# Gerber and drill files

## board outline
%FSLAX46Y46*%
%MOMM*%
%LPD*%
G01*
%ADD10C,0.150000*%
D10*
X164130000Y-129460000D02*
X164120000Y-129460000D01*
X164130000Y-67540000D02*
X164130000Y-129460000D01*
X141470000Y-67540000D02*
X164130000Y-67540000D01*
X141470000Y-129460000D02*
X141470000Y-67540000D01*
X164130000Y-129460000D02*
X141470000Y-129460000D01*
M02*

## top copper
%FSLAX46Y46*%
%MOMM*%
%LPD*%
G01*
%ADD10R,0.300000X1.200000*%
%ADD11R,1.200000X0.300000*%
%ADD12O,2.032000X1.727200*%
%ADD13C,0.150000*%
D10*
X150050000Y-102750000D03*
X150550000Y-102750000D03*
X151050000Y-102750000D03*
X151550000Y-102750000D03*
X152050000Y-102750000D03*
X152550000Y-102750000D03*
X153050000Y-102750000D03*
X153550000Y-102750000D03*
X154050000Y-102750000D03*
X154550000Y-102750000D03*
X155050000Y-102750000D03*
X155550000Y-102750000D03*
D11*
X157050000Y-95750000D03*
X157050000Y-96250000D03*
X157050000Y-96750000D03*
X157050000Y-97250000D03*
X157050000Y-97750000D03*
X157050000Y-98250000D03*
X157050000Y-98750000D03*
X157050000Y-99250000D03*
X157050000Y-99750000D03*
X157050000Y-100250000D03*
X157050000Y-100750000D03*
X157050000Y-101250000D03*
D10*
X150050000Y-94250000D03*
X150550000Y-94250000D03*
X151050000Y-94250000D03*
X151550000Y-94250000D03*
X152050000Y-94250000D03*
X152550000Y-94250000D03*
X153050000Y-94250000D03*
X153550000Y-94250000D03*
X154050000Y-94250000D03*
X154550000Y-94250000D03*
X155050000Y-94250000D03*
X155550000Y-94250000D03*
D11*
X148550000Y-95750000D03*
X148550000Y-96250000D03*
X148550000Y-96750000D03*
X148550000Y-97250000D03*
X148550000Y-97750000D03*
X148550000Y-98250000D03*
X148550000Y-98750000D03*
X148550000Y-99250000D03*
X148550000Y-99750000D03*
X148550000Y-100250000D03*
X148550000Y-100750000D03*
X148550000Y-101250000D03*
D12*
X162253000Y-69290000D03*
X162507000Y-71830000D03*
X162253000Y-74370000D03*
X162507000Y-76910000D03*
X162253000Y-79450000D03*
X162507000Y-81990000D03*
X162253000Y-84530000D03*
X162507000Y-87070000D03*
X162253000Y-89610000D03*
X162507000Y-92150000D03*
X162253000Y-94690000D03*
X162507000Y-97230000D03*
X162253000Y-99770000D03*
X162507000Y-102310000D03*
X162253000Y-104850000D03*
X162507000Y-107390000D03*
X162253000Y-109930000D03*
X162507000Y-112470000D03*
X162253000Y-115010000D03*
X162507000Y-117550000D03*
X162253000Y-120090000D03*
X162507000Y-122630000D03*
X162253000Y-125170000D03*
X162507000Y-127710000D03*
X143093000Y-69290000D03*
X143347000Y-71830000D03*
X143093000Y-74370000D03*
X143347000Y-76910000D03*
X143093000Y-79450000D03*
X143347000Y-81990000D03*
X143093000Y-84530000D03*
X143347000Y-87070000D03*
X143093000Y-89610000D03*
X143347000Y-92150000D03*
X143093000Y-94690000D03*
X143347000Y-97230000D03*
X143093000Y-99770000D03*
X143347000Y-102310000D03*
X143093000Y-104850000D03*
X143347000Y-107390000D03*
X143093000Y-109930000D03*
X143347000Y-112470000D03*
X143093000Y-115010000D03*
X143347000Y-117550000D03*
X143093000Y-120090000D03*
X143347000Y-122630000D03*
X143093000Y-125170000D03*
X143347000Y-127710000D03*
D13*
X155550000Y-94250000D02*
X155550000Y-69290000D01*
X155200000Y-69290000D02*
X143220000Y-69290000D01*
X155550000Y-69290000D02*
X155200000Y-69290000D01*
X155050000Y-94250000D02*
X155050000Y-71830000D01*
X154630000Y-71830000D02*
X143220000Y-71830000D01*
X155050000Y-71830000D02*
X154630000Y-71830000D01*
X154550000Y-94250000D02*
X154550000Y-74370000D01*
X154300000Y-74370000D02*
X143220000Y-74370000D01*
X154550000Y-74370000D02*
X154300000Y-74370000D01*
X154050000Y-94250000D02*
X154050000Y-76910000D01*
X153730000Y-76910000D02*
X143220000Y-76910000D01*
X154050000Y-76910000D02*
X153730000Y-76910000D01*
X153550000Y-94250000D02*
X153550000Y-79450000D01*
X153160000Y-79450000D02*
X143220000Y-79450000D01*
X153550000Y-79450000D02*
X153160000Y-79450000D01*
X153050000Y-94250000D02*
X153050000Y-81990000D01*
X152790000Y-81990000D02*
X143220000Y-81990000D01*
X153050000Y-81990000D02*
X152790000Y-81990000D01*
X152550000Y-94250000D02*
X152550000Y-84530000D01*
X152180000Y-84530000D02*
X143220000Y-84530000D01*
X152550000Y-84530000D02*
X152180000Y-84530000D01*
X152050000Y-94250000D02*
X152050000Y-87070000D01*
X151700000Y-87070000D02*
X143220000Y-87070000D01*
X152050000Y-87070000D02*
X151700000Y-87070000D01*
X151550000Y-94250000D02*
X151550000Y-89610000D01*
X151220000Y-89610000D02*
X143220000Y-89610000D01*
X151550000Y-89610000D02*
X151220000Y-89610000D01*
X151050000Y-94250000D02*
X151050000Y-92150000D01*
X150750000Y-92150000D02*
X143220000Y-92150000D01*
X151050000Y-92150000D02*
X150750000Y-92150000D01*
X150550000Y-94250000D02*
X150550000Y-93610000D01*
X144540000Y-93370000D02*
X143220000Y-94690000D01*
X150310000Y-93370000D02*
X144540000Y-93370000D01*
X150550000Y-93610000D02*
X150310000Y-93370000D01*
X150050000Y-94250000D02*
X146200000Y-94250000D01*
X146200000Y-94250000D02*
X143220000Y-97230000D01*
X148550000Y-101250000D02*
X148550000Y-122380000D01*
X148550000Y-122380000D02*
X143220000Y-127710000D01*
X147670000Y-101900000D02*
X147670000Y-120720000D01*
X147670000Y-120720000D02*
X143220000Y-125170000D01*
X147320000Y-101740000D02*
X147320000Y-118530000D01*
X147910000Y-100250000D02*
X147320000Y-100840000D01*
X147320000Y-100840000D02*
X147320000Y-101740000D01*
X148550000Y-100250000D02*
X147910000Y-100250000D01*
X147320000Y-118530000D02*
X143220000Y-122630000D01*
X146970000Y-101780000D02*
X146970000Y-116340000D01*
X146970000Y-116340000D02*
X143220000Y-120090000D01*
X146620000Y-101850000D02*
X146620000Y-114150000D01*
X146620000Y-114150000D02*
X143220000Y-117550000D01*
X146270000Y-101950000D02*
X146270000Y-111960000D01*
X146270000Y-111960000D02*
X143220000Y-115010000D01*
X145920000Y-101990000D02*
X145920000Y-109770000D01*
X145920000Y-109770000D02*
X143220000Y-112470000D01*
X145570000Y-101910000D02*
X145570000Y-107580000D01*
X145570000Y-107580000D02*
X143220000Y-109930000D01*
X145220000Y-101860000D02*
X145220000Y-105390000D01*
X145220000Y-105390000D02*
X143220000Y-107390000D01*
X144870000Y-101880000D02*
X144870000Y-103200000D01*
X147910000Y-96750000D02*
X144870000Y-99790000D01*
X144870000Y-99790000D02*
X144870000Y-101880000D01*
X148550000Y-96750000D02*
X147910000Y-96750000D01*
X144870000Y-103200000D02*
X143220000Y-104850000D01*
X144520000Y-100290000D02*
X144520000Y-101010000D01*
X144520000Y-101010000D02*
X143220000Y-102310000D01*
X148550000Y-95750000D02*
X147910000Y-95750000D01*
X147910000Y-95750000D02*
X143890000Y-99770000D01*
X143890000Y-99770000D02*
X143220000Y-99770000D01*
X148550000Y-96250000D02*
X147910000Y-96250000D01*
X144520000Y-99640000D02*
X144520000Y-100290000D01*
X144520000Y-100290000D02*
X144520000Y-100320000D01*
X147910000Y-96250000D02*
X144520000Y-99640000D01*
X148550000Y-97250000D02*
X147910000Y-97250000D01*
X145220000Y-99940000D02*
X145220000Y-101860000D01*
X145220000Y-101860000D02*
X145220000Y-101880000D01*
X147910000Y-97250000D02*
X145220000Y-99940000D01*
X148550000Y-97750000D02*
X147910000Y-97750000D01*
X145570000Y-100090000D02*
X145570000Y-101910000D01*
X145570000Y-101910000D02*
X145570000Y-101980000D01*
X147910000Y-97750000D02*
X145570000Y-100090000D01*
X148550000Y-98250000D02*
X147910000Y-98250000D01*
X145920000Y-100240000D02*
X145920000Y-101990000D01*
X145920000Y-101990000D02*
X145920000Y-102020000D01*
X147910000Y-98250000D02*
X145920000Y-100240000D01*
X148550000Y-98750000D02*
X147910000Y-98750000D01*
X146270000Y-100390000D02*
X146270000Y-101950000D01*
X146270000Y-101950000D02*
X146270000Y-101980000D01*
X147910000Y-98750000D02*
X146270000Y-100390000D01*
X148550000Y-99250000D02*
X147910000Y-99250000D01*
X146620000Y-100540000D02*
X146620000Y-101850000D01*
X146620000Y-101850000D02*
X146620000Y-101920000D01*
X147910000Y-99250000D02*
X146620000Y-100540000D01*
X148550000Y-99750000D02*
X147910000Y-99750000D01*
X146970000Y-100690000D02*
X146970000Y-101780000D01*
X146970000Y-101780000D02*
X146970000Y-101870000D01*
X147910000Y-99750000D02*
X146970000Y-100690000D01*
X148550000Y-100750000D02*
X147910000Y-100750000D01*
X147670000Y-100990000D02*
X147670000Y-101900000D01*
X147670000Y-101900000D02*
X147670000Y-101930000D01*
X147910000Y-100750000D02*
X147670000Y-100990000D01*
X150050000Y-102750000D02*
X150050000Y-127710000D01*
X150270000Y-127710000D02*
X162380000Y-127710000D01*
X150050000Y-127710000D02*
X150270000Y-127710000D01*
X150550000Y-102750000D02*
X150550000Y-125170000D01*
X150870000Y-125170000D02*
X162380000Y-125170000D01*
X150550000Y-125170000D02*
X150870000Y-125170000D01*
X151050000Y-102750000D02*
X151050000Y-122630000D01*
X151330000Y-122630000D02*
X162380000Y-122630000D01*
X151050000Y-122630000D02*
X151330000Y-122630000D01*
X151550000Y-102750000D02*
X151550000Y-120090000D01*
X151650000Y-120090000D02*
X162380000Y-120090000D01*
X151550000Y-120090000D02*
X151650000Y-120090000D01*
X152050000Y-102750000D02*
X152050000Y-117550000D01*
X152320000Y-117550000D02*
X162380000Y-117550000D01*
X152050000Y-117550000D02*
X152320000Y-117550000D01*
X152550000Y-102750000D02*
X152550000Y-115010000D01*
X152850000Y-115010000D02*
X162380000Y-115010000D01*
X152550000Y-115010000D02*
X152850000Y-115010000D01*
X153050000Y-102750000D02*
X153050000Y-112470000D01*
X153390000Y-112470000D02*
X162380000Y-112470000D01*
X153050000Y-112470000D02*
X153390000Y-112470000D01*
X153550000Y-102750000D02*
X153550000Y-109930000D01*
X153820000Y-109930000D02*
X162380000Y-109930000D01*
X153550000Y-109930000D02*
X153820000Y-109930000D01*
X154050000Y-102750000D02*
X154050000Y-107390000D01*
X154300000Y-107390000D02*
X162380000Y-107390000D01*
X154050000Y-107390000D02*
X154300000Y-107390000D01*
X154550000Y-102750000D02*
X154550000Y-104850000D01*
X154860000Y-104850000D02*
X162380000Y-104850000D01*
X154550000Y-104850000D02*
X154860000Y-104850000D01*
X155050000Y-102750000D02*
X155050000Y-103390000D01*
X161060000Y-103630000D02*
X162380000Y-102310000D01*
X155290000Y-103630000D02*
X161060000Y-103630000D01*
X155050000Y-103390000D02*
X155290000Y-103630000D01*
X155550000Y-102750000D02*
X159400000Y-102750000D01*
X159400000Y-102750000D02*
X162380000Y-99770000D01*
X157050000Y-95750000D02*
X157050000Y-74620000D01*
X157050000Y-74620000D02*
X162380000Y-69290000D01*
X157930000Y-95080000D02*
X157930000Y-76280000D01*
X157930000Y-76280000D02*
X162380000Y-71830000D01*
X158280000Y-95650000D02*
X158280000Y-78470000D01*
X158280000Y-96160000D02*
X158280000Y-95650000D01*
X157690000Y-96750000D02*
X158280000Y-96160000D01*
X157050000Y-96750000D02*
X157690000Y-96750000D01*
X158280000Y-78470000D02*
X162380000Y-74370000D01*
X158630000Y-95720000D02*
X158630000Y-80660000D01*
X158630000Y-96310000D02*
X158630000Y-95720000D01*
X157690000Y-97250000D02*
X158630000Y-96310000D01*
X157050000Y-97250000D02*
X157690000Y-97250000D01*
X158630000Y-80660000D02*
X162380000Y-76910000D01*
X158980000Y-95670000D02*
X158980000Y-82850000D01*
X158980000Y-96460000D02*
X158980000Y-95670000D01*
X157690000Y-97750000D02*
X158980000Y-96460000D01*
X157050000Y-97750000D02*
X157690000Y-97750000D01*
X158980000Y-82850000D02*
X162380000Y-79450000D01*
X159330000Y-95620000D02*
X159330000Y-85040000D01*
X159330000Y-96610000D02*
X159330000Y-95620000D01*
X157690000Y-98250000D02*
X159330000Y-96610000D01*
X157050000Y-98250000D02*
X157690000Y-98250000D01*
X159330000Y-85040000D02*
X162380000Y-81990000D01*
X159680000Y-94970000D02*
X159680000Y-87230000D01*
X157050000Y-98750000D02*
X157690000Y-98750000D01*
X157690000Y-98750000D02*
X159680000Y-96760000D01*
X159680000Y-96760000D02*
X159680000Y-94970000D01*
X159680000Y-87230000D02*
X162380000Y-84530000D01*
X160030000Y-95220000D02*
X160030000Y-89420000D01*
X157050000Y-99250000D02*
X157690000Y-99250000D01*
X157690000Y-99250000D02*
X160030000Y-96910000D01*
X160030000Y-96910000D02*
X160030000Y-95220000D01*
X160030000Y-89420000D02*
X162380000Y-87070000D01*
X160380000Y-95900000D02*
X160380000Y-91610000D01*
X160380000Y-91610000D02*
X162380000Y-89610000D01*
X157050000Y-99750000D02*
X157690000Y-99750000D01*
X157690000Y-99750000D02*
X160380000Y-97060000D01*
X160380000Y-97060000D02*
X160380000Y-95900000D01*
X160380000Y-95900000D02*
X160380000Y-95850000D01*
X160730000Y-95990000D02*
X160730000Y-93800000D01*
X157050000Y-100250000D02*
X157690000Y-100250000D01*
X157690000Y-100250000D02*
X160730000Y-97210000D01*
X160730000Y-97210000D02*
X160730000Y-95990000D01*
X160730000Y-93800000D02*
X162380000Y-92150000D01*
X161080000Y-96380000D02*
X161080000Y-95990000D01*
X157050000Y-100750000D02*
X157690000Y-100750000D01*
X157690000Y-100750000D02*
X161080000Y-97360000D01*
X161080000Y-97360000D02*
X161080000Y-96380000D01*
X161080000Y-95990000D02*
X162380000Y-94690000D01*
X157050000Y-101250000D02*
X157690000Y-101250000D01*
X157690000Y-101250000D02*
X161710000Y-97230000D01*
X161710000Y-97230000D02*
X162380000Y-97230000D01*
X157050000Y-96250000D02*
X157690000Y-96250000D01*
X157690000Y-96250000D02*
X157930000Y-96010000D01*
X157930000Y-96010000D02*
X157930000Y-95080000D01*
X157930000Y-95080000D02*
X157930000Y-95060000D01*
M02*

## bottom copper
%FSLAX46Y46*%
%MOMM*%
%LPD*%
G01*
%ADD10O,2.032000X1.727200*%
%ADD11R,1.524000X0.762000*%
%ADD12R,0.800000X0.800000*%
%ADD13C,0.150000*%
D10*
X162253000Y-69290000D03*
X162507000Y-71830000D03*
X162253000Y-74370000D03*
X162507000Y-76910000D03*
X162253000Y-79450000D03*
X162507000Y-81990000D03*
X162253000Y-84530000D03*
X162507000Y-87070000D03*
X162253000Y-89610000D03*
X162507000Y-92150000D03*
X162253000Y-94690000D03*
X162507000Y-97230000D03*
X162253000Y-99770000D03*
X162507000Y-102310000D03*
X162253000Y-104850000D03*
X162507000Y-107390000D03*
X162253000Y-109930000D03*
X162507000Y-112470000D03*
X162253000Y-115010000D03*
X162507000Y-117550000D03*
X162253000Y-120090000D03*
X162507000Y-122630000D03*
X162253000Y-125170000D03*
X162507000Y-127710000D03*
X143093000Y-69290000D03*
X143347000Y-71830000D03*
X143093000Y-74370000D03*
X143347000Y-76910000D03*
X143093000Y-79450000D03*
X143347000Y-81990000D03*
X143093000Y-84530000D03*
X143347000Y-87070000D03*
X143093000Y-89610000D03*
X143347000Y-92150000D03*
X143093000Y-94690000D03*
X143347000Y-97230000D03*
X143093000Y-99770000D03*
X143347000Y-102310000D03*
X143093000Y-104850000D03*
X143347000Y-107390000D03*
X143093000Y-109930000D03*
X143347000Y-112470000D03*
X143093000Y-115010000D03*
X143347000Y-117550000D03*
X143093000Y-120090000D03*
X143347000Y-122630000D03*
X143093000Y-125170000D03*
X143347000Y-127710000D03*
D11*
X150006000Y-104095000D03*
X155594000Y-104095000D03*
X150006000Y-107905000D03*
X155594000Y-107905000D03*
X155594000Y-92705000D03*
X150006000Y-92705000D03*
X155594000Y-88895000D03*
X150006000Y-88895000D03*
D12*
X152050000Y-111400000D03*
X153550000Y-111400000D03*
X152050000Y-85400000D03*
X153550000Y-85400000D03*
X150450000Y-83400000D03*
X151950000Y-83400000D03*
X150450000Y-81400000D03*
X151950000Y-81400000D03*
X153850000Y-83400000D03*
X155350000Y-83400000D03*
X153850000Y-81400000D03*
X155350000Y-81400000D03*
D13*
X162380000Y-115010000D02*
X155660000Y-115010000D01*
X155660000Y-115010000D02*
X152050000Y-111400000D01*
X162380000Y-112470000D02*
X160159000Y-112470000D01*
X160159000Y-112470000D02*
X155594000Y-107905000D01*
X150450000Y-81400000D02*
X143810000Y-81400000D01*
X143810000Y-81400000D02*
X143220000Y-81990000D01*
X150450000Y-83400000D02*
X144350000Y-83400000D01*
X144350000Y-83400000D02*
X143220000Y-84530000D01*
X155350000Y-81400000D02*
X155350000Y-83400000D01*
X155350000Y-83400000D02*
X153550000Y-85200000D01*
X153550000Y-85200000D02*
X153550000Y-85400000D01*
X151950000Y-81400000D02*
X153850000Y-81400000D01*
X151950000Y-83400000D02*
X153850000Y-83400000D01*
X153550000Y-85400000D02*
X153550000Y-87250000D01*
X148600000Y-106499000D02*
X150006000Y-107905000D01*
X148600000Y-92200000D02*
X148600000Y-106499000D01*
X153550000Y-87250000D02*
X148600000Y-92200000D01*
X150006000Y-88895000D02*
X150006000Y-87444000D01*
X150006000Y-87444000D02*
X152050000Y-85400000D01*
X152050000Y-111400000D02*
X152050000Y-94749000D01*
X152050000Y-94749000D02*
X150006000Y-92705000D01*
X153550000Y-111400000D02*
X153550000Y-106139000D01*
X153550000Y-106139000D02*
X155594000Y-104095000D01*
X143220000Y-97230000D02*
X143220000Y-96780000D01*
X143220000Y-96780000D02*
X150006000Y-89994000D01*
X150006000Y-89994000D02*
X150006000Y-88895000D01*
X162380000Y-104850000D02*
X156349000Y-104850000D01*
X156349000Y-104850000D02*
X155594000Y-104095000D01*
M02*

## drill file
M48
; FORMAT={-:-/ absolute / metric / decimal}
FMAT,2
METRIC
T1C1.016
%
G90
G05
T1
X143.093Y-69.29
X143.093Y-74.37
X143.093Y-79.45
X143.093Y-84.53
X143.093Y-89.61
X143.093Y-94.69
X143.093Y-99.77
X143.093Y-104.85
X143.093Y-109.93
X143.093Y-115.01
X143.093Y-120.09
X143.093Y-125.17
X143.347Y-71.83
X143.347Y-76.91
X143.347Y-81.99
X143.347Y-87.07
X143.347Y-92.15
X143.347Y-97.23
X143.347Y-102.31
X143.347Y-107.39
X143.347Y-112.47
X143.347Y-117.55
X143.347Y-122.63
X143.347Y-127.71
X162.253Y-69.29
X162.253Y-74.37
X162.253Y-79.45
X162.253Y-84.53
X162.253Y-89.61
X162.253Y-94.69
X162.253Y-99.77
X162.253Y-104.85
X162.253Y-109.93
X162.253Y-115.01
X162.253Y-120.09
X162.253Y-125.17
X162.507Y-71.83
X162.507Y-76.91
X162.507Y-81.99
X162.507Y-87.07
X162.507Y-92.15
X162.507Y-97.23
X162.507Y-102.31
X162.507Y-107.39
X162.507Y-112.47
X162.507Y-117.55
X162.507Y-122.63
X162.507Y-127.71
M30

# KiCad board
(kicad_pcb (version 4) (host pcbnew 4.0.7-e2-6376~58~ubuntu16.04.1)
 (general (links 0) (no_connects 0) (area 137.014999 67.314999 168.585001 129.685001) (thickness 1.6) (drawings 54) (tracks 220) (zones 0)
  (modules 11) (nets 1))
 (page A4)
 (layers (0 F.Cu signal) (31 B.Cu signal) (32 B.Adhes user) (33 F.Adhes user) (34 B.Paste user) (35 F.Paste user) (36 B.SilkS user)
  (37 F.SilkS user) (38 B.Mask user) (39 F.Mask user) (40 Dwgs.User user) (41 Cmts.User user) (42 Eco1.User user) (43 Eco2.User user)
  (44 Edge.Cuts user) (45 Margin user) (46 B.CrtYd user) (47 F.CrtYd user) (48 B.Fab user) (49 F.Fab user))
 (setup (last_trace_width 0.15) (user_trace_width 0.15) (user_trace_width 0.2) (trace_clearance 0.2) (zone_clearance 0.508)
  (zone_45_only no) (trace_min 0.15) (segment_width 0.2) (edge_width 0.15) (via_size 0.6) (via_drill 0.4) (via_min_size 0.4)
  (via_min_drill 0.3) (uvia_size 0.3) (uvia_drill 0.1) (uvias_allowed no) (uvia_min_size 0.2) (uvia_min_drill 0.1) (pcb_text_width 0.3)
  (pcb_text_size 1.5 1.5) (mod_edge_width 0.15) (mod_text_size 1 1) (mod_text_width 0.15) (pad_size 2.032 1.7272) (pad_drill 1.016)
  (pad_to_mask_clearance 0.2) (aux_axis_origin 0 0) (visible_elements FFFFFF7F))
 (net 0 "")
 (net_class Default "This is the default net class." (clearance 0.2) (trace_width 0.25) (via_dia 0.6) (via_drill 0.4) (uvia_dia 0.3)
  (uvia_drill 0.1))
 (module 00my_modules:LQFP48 (layer F.Cu) (at 152.8 98.5)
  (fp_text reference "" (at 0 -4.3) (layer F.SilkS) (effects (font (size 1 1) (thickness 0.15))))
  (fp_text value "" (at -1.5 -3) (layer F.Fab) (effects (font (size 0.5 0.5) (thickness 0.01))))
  (pad 1 smd rect (at -2.75 4.25) (size 0.3 1.2) (layers F.Cu F.Paste F.Mask))
  (pad 2 smd rect (at -2.25 4.25) (size 0.3 1.2) (layers F.Cu F.Paste F.Mask))
  (pad 3 smd rect (at -1.75 4.25) (size 0.3 1.2) (layers F.Cu F.Paste F.Mask))
  (pad 4 smd rect (at -1.25 4.25) (size 0.3 1.2) (layers F.Cu F.Paste F.Mask))
  (pad 5 smd rect (at -0.75 4.25) (size 0.3 1.2) (layers F.Cu F.Paste F.Mask))
  (pad 6 smd rect (at -0.25 4.25) (size 0.3 1.2) (layers F.Cu F.Paste F.Mask))
  (pad 7 smd rect (at 0.25 4.25) (size 0.3 1.2) (layers F.Cu F.Paste F.Mask))
  (pad 8 smd rect (at 0.75 4.25) (size 0.3 1.2) (layers F.Cu F.Paste F.Mask))
  (pad 9 smd rect (at 1.25 4.25) (size 0.3 1.2) (layers F.Cu F.Paste F.Mask))
  (pad 10 smd rect (at 1.75 4.25) (size 0.3 1.2) (layers F.Cu F.Paste F.Mask))
  (pad 11 smd rect (at 2.25 4.25) (size 0.3 1.2) (layers F.Cu F.Paste F.Mask))
  (pad 12 smd rect (at 2.75 4.25) (size 0.3 1.2) (layers F.Cu F.Paste F.Mask))
  (pad 24 smd rect (at 4.25 -2.75) (size 1.2 0.3) (layers F.Cu F.Paste F.Mask))
  (pad 23 smd rect (at 4.25 -2.25) (size 1.2 0.3) (layers F.Cu F.Paste F.Mask))
  (pad 22 smd rect (at 4.25 -1.75) (size 1.2 0.3) (layers F.Cu F.Paste F.Mask))
  (pad 21 smd rect (at 4.25 -1.25) (size 1.2 0.3) (layers F.Cu F.Paste F.Mask))
  (pad 20 smd rect (at 4.25 -0.75) (size 1.2 0.3) (layers F.Cu F.Paste F.Mask))
  (pad 19 smd rect (at 4.25 -0.25) (size 1.2 0.3) (layers F.Cu F.Paste F.Mask))
  (pad 18 smd rect (at 4.25 0.25) (size 1.2 0.3) (layers F.Cu F.Paste F.Mask))
  (pad 17 smd rect (at 4.25 0.75) (size 1.2 0.3) (layers F.Cu F.Paste F.Mask))
  (pad 16 smd rect (at 4.25 1.25) (size 1.2 0.3) (layers F.Cu F.Paste F.Mask))
  (pad 15 smd rect (at 4.25 1.75) (size 1.2 0.3) (layers F.Cu F.Paste F.Mask))
  (pad 14 smd rect (at 4.25 2.25) (size 1.2 0.3) (layers F.Cu F.Paste F.Mask))
  (pad 13 smd rect (at 4.25 2.75) (size 1.2 0.3) (layers F.Cu F.Paste F.Mask))
  (pad 36 smd rect (at -2.75 -4.25) (size 0.3 1.2) (layers F.Cu F.Paste F.Mask))
  (pad 35 smd rect (at -2.25 -4.25) (size 0.3 1.2) (layers F.Cu F.Paste F.Mask))
  (pad 34 smd rect (at -1.75 -4.25) (size 0.3 1.2) (layers F.Cu F.Paste F.Mask))
  (pad 33 smd rect (at -1.25 -4.25) (size 0.3 1.2) (layers F.Cu F.Paste F.Mask))
  (pad 32 smd rect (at -0.75 -4.25) (size 0.3 1.2) (layers F.Cu F.Paste F.Mask))
  (pad 31 smd rect (at -0.25 -4.25) (size 0.3 1.2) (layers F.Cu F.Paste F.Mask))
  (pad 30 smd rect (at 0.25 -4.25) (size 0.3 1.2) (layers F.Cu F.Paste F.Mask))
  (pad 29 smd rect (at 0.75 -4.25) (size 0.3 1.2) (layers F.Cu F.Paste F.Mask))
  (pad 28 smd rect (at 1.25 -4.25) (size 0.3 1.2) (layers F.Cu F.Paste F.Mask))
  (pad 27 smd rect (at 1.75 -4.25) (size 0.3 1.2) (layers F.Cu F.Paste F.Mask))
  (pad 26 smd rect (at 2.25 -4.25) (size 0.3 1.2) (layers F.Cu F.Paste F.Mask))
  (pad 25 smd rect (at 2.75 -4.25) (size 0.3 1.2) (layers F.Cu F.Paste F.Mask))
  (pad 37 smd rect (at -4.25 -2.75) (size 1.2 0.3) (layers F.Cu F.Paste F.Mask))
  (pad 38 smd rect (at -4.25 -2.25) (size 1.2 0.3) (layers F.Cu F.Paste F.Mask))
  (pad 39 smd rect (at -4.25 -1.75) (size 1.2 0.3) (layers F.Cu F.Paste F.Mask))
  (pad 40 smd rect (at -4.25 -1.25) (size 1.2 0.3) (layers F.Cu F.Paste F.Mask))
  (pad 41 smd rect (at -4.25 -0.75) (size 1.2 0.3) (layers F.Cu F.Paste F.Mask))
  (pad 42 smd rect (at -4.25 -0.25) (size 1.2 0.3) (layers F.Cu F.Paste F.Mask))
  (pad 43 smd rect (at -4.25 0.25) (size 1.2 0.3) (layers F.Cu F.Paste F.Mask))
  (pad 44 smd rect (at -4.25 0.75) (size 1.2 0.3) (layers F.Cu F.Paste F.Mask))
  (pad 45 smd rect (at -4.25 1.25) (size 1.2 0.3) (layers F.Cu F.Paste F.Mask))
  (pad 46 smd rect (at -4.25 1.75) (size 1.2 0.3) (layers F.Cu F.Paste F.Mask))
  (pad 47 smd rect (at -4.25 2.25) (size 1.2 0.3) (layers F.Cu F.Paste F.Mask))
  (pad 48 smd rect (at -4.25 2.75) (size 1.2 0.3) (layers F.Cu F.Paste F.Mask)))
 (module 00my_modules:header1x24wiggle (layer F.Cu) (at 162.38 98.5)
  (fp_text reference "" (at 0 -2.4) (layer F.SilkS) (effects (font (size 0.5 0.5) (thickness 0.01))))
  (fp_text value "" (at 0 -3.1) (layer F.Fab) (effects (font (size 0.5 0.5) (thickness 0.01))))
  (pad 24 thru_hole oval (at -0.127 -29.21) (size 2.032 1.7272) (drill 1.016) (layers *.Cu *.Mask F.SilkS))
  (pad 23 thru_hole oval (at 0.127 -26.67) (size 2.032 1.7272) (drill 1.016) (layers *.Cu *.Mask F.SilkS))
  (pad 22 thru_hole oval (at -0.127 -24.13) (size 2.032 1.7272) (drill 1.016) (layers *.Cu *.Mask F.SilkS))
  (pad 21 thru_hole oval (at 0.127 -21.59) (size 2.032 1.7272) (drill 1.016) (layers *.Cu *.Mask F.SilkS))
  (pad 20 thru_hole oval (at -0.127 -19.05) (size 2.032 1.7272) (drill 1.016) (layers *.Cu *.Mask F.SilkS))
  (pad 19 thru_hole oval (at 0.127 -16.51) (size 2.032 1.7272) (drill 1.016) (layers *.Cu *.Mask F.SilkS))
  (pad 18 thru_hole oval (at -0.127 -13.97) (size 2.032 1.7272) (drill 1.016) (layers *.Cu *.Mask F.SilkS))
  (pad 17 thru_hole oval (at 0.127 -11.43) (size 2.032 1.7272) (drill 1.016) (layers *.Cu *.Mask F.SilkS))
  (pad 16 thru_hole oval (at -0.127 -8.89) (size 2.032 1.7272) (drill 1.016) (layers *.Cu *.Mask F.SilkS))
  (pad 15 thru_hole oval (at 0.127 -6.35) (size 2.032 1.7272) (drill 1.016) (layers *.Cu *.Mask F.SilkS))
  (pad 14 thru_hole oval (at -0.127 -3.81) (size 2.032 1.7272) (drill 1.016) (layers *.Cu *.Mask F.SilkS))
  (pad 13 thru_hole oval (at 0.127 -1.27) (size 2.032 1.7272) (drill 1.016) (layers *.Cu *.Mask F.SilkS))
  (pad 12 thru_hole oval (at -0.127 1.27) (size 2.032 1.7272) (drill 1.016) (layers *.Cu *.Mask F.SilkS))
  (pad 11 thru_hole oval (at 0.127 3.81) (size 2.032 1.7272) (drill 1.016) (layers *.Cu *.Mask F.SilkS))
  (pad 10 thru_hole oval (at -0.127 6.35) (size 2.032 1.7272) (drill 1.016) (layers *.Cu *.Mask F.SilkS))
  (pad 9 thru_hole oval (at 0.127 8.89) (size 2.032 1.7272) (drill 1.016) (layers *.Cu *.Mask F.SilkS))
  (pad 8 thru_hole oval (at -0.127 11.43) (size 2.032 1.7272) (drill 1.016) (layers *.Cu *.Mask F.SilkS))
  (pad 7 thru_hole oval (at 0.127 13.97) (size 2.032 1.7272) (drill 1.016) (layers *.Cu *.Mask F.SilkS))
  (pad 6 thru_hole oval (at -0.127 16.51) (size 2.032 1.7272) (drill 1.016) (layers *.Cu *.Mask F.SilkS))
  (pad 5 thru_hole oval (at 0.127 19.05) (size 2.032 1.7272) (drill 1.016) (layers *.Cu *.Mask F.SilkS))
  (pad 4 thru_hole oval (at -0.127 21.59) (size 2.032 1.7272) (drill 1.016) (layers *.Cu *.Mask F.SilkS))
  (pad 3 thru_hole oval (at 0.127 24.13) (size 2.032 1.7272) (drill 1.016) (layers *.Cu *.Mask F.SilkS))
  (pad 2 thru_hole oval (at -0.127 26.67) (size 2.032 1.7272) (drill 1.016) (layers *.Cu *.Mask F.SilkS))
  (pad 1 thru_hole oval (at 0.127 29.21) (size 2.032 1.7272) (drill 1.016) (layers *.Cu *.Mask F.SilkS)))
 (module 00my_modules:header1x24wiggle (layer F.Cu) (at 143.22 98.5)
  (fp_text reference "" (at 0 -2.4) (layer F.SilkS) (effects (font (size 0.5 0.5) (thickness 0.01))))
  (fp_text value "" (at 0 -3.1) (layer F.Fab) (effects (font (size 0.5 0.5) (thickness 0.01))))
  (pad 25 thru_hole oval (at -0.127 -29.21) (size 2.032 1.7272) (drill 1.016) (layers *.Cu *.Mask F.SilkS))
  (pad 26 thru_hole oval (at 0.127 -26.67) (size 2.032 1.7272) (drill 1.016) (layers *.Cu *.Mask F.SilkS))
  (pad 27 thru_hole oval (at -0.127 -24.13) (size 2.032 1.7272) (drill 1.016) (layers *.Cu *.Mask F.SilkS))
  (pad 28 thru_hole oval (at 0.127 -21.59) (size 2.032 1.7272) (drill 1.016) (layers *.Cu *.Mask F.SilkS))
  (pad 29 thru_hole oval (at -0.127 -19.05) (size 2.032 1.7272) (drill 1.016) (layers *.Cu *.Mask F.SilkS))
  (pad 30 thru_hole oval (at 0.127 -16.51) (size 2.032 1.7272) (drill 1.016) (layers *.Cu *.Mask F.SilkS))
  (pad 31 thru_hole oval (at -0.127 -13.97) (size 2.032 1.7272) (drill 1.016) (layers *.Cu *.Mask F.SilkS))
  (pad 32 thru_hole oval (at 0.127 -11.43) (size 2.032 1.7272) (drill 1.016) (layers *.Cu *.Mask F.SilkS))
  (pad 33 thru_hole oval (at -0.127 -8.89) (size 2.032 1.7272) (drill 1.016) (layers *.Cu *.Mask F.SilkS))
  (pad 34 thru_hole oval (at 0.127 -6.35) (size 2.032 1.7272) (drill 1.016) (layers *.Cu *.Mask F.SilkS))
  (pad 35 thru_hole oval (at -0.127 -3.81) (size 2.032 1.7272) (drill 1.016) (layers *.Cu *.Mask F.SilkS))
  (pad 36 thru_hole oval (at 0.127 -1.27) (size 2.032 1.7272) (drill 1.016) (layers *.Cu *.Mask F.SilkS))
  (pad 37 thru_hole oval (at -0.127 1.27) (size 2.032 1.7272) (drill 1.016) (layers *.Cu *.Mask F.SilkS))
  (pad 38 thru_hole oval (at 0.127 3.81) (size 2.032 1.7272) (drill 1.016) (layers *.Cu *.Mask F.SilkS))
  (pad 39 thru_hole oval (at -0.127 6.35) (size 2.032 1.7272) (drill 1.016) (layers *.Cu *.Mask F.SilkS))
  (pad 40 thru_hole oval (at 0.127 8.89) (size 2.032 1.7272) (drill 1.016) (layers *.Cu *.Mask F.SilkS))
  (pad 41 thru_hole oval (at -0.127 11.43) (size 2.032 1.7272) (drill 1.016) (layers *.Cu *.Mask F.SilkS))
  (pad 42 thru_hole oval (at 0.127 13.97) (size 2.032 1.7272) (drill 1.016) (layers *.Cu *.Mask F.SilkS))
  (pad 43 thru_hole oval (at -0.127 16.51) (size 2.032 1.7272) (drill 1.016) (layers *.Cu *.Mask F.SilkS))
  (pad 44 thru_hole oval (at 0.127 19.05) (size 2.032 1.7272) (drill 1.016) (layers *.Cu *.Mask F.SilkS))
  (pad 45 thru_hole oval (at -0.127 21.59) (size 2.032 1.7272) (drill 1.016) (layers *.Cu *.Mask F.SilkS))
  (pad 46 thru_hole oval (at 0.127 24.13) (size 2.032 1.7272) (drill 1.016) (layers *.Cu *.Mask F.SilkS))
  (pad 47 thru_hole oval (at -0.127 26.67) (size 2.032 1.7272) (drill 1.016) (layers *.Cu *.Mask F.SilkS))
  (pad 48 thru_hole oval (at 0.127 29.21) (size 2.032 1.7272) (drill 1.016) (layers *.Cu *.Mask F.SilkS)))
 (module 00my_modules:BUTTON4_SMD (layer B.Cu) (at 152.8 106)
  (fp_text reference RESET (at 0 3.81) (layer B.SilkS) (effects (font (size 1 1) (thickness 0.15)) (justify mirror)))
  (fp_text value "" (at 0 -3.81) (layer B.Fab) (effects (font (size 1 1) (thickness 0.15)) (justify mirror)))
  (pad 1 smd rect (at -2.794 -1.905) (size 1.524 0.762) (layers B.Cu B.Paste B.Mask))
  (pad 2 smd rect (at 2.794 -1.905) (size 1.524 0.762) (layers B.Cu B.Paste B.Mask))
  (pad 3 smd rect (at -2.794 1.905) (size 1.524 0.762) (layers B.Cu B.Paste B.Mask))
  (pad 4 smd rect (at 2.794 1.905) (size 1.524 0.762) (layers B.Cu B.Paste B.Mask)))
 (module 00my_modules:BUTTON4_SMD (layer B.Cu) (at 152.8 90.8 180)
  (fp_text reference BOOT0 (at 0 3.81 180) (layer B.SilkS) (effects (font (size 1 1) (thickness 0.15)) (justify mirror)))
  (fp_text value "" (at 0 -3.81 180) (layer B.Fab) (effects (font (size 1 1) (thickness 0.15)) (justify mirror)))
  (pad 1 smd rect (at -2.794 -1.905 180) (size 1.524 0.762) (layers B.Cu B.Paste B.Mask))
  (pad 2 smd rect (at 2.794 -1.905 180) (size 1.524 0.762) (layers B.Cu B.Paste B.Mask))
  (pad 3 smd rect (at -2.794 1.905 180) (size 1.524 0.762) (layers B.Cu B.Paste B.Mask))
  (pad 4 smd rect (at 2.794 1.905 180) (size 1.524 0.762) (layers B.Cu B.Paste B.Mask)))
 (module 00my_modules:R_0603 (layer B.Cu) (at 152.8 111.4)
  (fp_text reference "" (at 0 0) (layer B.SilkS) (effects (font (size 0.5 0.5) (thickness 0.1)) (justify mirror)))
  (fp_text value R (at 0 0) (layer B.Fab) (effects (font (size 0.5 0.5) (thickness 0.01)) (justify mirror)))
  (pad 1 smd rect (at -0.75 0) (size 0.8 0.8) (layers B.Cu B.Paste B.Mask))
  (pad 2 smd rect (at 0.75 0) (size 0.8 0.8) (layers B.Cu B.Paste B.Mask)))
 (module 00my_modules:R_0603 (layer B.Cu) (at 152.8 85.4)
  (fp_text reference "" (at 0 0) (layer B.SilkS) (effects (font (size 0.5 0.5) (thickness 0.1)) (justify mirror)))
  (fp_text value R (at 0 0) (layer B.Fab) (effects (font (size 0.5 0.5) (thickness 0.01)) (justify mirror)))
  (pad 1 smd rect (at -0.75 0) (size 0.8 0.8) (layers B.Cu B.Paste B.Mask))
  (pad 2 smd rect (at 0.75 0) (size 0.8 0.8) (layers B.Cu B.Paste B.Mask)))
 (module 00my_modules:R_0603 (layer B.Cu) (at 151.2 83.4)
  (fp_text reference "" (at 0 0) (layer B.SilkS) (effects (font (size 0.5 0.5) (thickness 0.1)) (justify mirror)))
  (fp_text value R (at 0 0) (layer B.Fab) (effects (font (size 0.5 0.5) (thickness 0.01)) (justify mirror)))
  (pad 1 smd rect (at -0.75 0) (size 0.8 0.8) (layers B.Cu B.Paste B.Mask))
  (pad 2 smd rect (at 0.75 0) (size 0.8 0.8) (layers B.Cu B.Paste B.Mask)))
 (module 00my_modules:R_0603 (layer B.Cu) (at 151.2 81.4)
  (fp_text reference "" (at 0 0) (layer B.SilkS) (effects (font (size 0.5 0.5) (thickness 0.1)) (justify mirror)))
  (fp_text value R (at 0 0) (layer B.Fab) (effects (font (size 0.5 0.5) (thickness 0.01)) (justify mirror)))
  (pad 1 smd rect (at -0.75 0) (size 0.8 0.8) (layers B.Cu B.Paste B.Mask))
  (pad 2 smd rect (at 0.75 0) (size 0.8 0.8) (layers B.Cu B.Paste B.Mask)))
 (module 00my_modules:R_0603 (layer B.Cu) (at 154.6 83.4)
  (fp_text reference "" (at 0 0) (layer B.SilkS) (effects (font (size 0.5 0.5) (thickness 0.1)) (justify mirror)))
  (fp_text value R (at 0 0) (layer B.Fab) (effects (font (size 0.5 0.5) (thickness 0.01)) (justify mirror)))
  (pad 1 smd rect (at -0.75 0) (size 0.8 0.8) (layers B.Cu B.Paste B.Mask))
  (pad 2 smd rect (at 0.75 0) (size 0.8 0.8) (layers B.Cu B.Paste B.Mask)))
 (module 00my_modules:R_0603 (layer B.Cu) (at 154.6 81.4)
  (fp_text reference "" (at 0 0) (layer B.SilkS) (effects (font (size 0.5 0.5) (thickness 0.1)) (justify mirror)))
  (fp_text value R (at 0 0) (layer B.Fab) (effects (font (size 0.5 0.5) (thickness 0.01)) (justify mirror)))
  (pad 1 smd rect (at -0.75 0) (size 0.8 0.8) (layers B.Cu B.Paste B.Mask))
  (pad 2 smd rect (at 0.75 0) (size 0.8 0.8) (layers B.Cu B.Paste B.Mask)))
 (gr_line (start 164.13 129.46) (end 164.12 129.46) (angle 90) (layer Edge.Cuts) (width 0.15))
 (gr_line (start 164.13 67.54) (end 164.13 129.46) (angle 90) (layer Edge.Cuts) (width 0.15))
 (gr_line (start 141.47 67.54) (end 164.13 67.54) (angle 90) (layer Edge.Cuts) (width 0.15))
 (gr_line (start 141.47 129.46) (end 141.47 67.54) (angle 90) (layer Edge.Cuts) (width 0.15))
 (gr_line (start 164.13 129.46) (end 141.47 129.46) (angle 90) (layer Edge.Cuts) (width 0.15))
 (segment (start 162.38 115.01) (end 155.66 115.01) (width 0.15) (layer B.Cu) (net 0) (status 400000))
 (segment (start 155.66 115.01) (end 152.05 111.4) (width 0.15) (layer B.Cu) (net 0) (status 800000))
 (segment (start 162.38 112.47) (end 160.159 112.47) (width 0.15) (layer B.Cu) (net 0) (status 400000))
 (segment (start 160.159 112.47) (end 155.594 107.905) (width 0.15) (layer B.Cu) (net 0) (status 800000))
 (segment (start 150.45 81.4) (end 143.81 81.4) (width 0.15) (layer B.Cu) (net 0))
 (segment (start 143.81 81.4) (end 143.22 81.99) (width 0.15) (layer B.Cu) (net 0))
 (segment (start 150.45 83.4) (end 144.35 83.4) (width 0.15) (layer B.Cu) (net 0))
 (segment (start 144.35 83.4) (end 143.22 84.53) (width 0.15) (layer B.Cu) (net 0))
 (segment (start 155.35 81.4) (end 155.35 83.4) (width 0.15) (layer B.Cu) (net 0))
 (segment (start 155.35 83.4) (end 153.55 85.2) (width 0.15) (layer B.Cu) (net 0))
 (segment (start 153.55 85.2) (end 153.55 85.4) (width 0.15) (layer B.Cu) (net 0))
 (segment (start 151.95 81.4) (end 153.85 81.4) (width 0.15) (layer B.Cu) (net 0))
 (segment (start 151.95 83.4) (end 153.85 83.4) (width 0.15) (layer B.Cu) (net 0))
 (segment (start 153.55 85.4) (end 153.55 87.25) (width 0.15) (layer B.Cu) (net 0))
 (segment (start 148.6 106.499) (end 150.006 107.905) (width 0.15) (layer B.Cu) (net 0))
 (segment (start 148.6 92.2) (end 148.6 106.499) (width 0.15) (layer B.Cu) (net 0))
 (segment (start 153.55 87.25) (end 148.6 92.2) (width 0.15) (layer B.Cu) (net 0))
 (segment (start 150.006 88.895) (end 150.006 87.444) (width 0.15) (layer B.Cu) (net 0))
 (segment (start 150.006 87.444) (end 152.05 85.4) (width 0.15) (layer B.Cu) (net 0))
 (segment (start 152.05 111.4) (end 152.05 94.749) (width 0.15) (layer B.Cu) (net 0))
 (segment (start 152.05 94.749) (end 150.006 92.705) (width 0.15) (layer B.Cu) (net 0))
 (segment (start 153.55 111.4) (end 153.55 106.139) (width 0.15) (layer B.Cu) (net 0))
 (segment (start 153.55 106.139) (end 155.594 104.095) (width 0.15) (layer B.Cu) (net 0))
 (segment (start 143.22 97.23) (end 143.22 96.78) (width 0.15) (layer B.Cu) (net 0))
 (segment (start 143.22 96.78) (end 150.006 89.994) (width 0.15) (layer B.Cu) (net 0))
 (segment (start 150.006 89.994) (end 150.006 88.895) (width 0.15) (layer B.Cu) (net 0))
 (segment (start 162.38 104.85) (end 156.349 104.85) (width 0.15) (layer B.Cu) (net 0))
 (segment (start 156.349 104.85) (end 155.594 104.095) (width 0.15) (layer B.Cu) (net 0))
 (segment (start 155.55 94.25) (end 155.55 69.29) (width 0.15) (layer F.Cu) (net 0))
 (segment (start 155.2 69.29) (end 143.22 69.29) (width 0.15) (layer F.Cu) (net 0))
 (segment (start 155.55 69.29) (end 155.2 69.29) (width 0.15) (layer F.Cu) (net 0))
 (segment (start 155.05 94.25) (end 155.05 71.83) (width 0.15) (layer F.Cu) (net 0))
 (segment (start 154.63 71.83) (end 143.22 71.83) (width 0.15) (layer F.Cu) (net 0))
 (segment (start 155.05 71.83) (end 154.63 71.83) (width 0.15) (layer F.Cu) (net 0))
 (segment (start 154.55 94.25) (end 154.55 74.37) (width 0.15) (layer F.Cu) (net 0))
 (segment (start 154.3 74.37) (end 143.22 74.37) (width 0.15) (layer F.Cu) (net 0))
 (segment (start 154.55 74.37) (end 154.3 74.37) (width 0.15) (layer F.Cu) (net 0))
 (segment (start 154.05 94.25) (end 154.05 76.91) (width 0.15) (layer F.Cu) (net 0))
 (segment (start 153.73 76.91) (end 143.22 76.91) (width 0.15) (layer F.Cu) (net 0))
 (segment (start 154.05 76.91) (end 153.73 76.91) (width 0.15) (layer F.Cu) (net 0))
 (segment (start 153.55 94.25) (end 153.55 79.45) (width 0.15) (layer F.Cu) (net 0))
 (segment (start 153.16 79.45) (end 143.22 79.45) (width 0.15) (layer F.Cu) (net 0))
 (segment (start 153.55 79.45) (end 153.16 79.45) (width 0.15) (layer F.Cu) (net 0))
 (segment (start 153.05 94.25) (end 153.05 81.99) (width 0.15) (layer F.Cu) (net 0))
 (segment (start 152.79 81.99) (end 143.22 81.99) (width 0.15) (layer F.Cu) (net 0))
 (segment (start 153.05 81.99) (end 152.79 81.99) (width 0.15) (layer F.Cu) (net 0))
 (segment (start 152.55 94.25) (end 152.55 84.53) (width 0.15) (layer F.Cu) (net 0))
 (segment (start 152.18 84.53) (end 143.22 84.53) (width 0.15) (layer F.Cu) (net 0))
 (segment (start 152.55 84.53) (end 152.18 84.53) (width 0.15) (layer F.Cu) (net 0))
 (segment (start 152.05 94.25) (end 152.05 87.07) (width 0.15) (layer F.Cu) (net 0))
 (segment (start 151.7 87.07) (end 143.22 87.07) (width 0.15) (layer F.Cu) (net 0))
 (segment (start 152.05 87.07) (end 151.7 87.07) (width 0.15) (layer F.Cu) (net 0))
 (segment (start 151.55 94.25) (end 151.55 89.61) (width 0.15) (layer F.Cu) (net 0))
 (segment (start 151.22 89.61) (end 143.22 89.61) (width 0.15) (layer F.Cu) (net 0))
 (segment (start 151.55 89.61) (end 151.22 89.61) (width 0.15) (layer F.Cu) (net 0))
 (segment (start 151.05 94.25) (end 151.05 92.15) (width 0.15) (layer F.Cu) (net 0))
 (segment (start 150.75 92.15) (end 143.22 92.15) (width 0.15) (layer F.Cu) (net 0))
 (segment (start 151.05 92.15) (end 150.75 92.15) (width 0.15) (layer F.Cu) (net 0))
 (segment (start 150.55 94.25) (end 150.55 93.61) (width 0.15) (layer F.Cu) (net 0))
 (segment (start 144.54 93.37) (end 143.22 94.69) (width 0.15) (layer F.Cu) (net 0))
 (segment (start 150.31 93.37) (end 144.54 93.37) (width 0.15) (layer F.Cu) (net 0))
 (segment (start 150.55 93.61) (end 150.31 93.37) (width 0.15) (layer F.Cu) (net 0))
 (segment (start 150.05 94.25) (end 146.2 94.25) (width 0.15) (layer F.Cu) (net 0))
 (segment (start 146.2 94.25) (end 143.22 97.23) (width 0.15) (layer F.Cu) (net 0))
 (segment (start 148.55 101.25) (end 148.55 122.38) (width 0.15) (layer F.Cu) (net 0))
 (segment (start 148.55 122.38) (end 143.22 127.71) (width 0.15) (layer F.Cu) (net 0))
 (segment (start 147.67 101.9) (end 147.67 120.72) (width 0.15) (layer F.Cu) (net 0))
 (segment (start 147.67 120.72) (end 143.22 125.17) (width 0.15) (layer F.Cu) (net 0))
 (segment (start 147.32 101.74) (end 147.32 118.53) (width 0.15) (layer F.Cu) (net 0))
 (segment (start 147.91 100.25) (end 147.32 100.84) (width 0.15) (layer F.Cu) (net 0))
 (segment (start 147.32 100.84) (end 147.32 101.74) (width 0.15) (layer F.Cu) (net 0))
 (segment (start 148.55 100.25) (end 147.91 100.25) (width 0.15) (layer F.Cu) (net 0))
 (segment (start 147.32 118.53) (end 143.22 122.63) (width 0.15) (layer F.Cu) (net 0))
 (segment (start 146.97 101.78) (end 146.97 116.34) (width 0.15) (layer F.Cu) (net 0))
 (segment (start 146.97 116.34) (end 143.22 120.09) (width 0.15) (layer F.Cu) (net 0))
 (segment (start 146.62 101.85) (end 146.62 114.15) (width 0.15) (layer F.Cu) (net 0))
 (segment (start 146.62 114.15) (end 143.22 117.55) (width 0.15) (layer F.Cu) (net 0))
 (segment (start 146.27 101.95) (end 146.27 111.96) (width 0.15) (layer F.Cu) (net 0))
 (segment (start 146.27 111.96) (end 143.22 115.01) (width 0.15) (layer F.Cu) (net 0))
 (segment (start 145.92 101.99) (end 145.92 109.77) (width 0.15) (layer F.Cu) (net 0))
 (segment (start 145.92 109.77) (end 143.22 112.47) (width 0.15) (layer F.Cu) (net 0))
 (segment (start 145.57 101.91) (end 145.57 107.58) (width 0.15) (layer F.Cu) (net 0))
 (segment (start 145.57 107.58) (end 143.22 109.93) (width 0.15) (layer F.Cu) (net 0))
 (segment (start 145.22 101.86) (end 145.22 105.39) (width 0.15) (layer F.Cu) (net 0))
 (segment (start 145.22 105.39) (end 143.22 107.39) (width 0.15) (layer F.Cu) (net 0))
 (segment (start 144.87 101.88) (end 144.87 103.2) (width 0.15) (layer F.Cu) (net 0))
 (segment (start 147.91 96.75) (end 144.87 99.79) (width 0.15) (layer F.Cu) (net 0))
 (segment (start 144.87 99.79) (end 144.87 101.88) (width 0.15) (layer F.Cu) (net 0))
 (segment (start 148.55 96.75) (end 147.91 96.75) (width 0.15) (layer F.Cu) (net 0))
 (segment (start 144.87 103.2) (end 143.22 104.85) (width 0.15) (layer F.Cu) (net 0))
 (segment (start 144.52 100.29) (end 144.52 101.01) (width 0.15) (layer F.Cu) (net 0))
 (segment (start 144.52 101.01) (end 143.22 102.31) (width 0.15) (layer F.Cu) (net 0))
 (segment (start 148.55 95.75) (end 147.91 95.75) (width 0.15) (layer F.Cu) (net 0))
 (segment (start 147.91 95.75) (end 143.89 99.77) (width 0.15) (layer F.Cu) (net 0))
 (segment (start 143.89 99.77) (end 143.22 99.77) (width 0.15) (layer F.Cu) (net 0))
 (segment (start 148.55 96.25) (end 147.91 96.25) (width 0.15) (layer F.Cu) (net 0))
 (segment (start 144.52 99.64) (end 144.52 100.29) (width 0.15) (layer F.Cu) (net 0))
 (segment (start 144.52 100.29) (end 144.52 100.32) (width 0.15) (layer F.Cu) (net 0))
 (segment (start 147.91 96.25) (end 144.52 99.64) (width 0.15) (layer F.Cu) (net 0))
 (segment (start 148.55 97.25) (end 147.91 97.25) (width 0.15) (layer F.Cu) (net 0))
 (segment (start 145.22 99.94) (end 145.22 101.86) (width 0.15) (layer F.Cu) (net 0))
 (segment (start 145.22 101.86) (end 145.22 101.88) (width 0.15) (layer F.Cu) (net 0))
 (segment (start 147.91 97.25) (end 145.22 99.94) (width 0.15) (layer F.Cu) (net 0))
 (segment (start 148.55 97.75) (end 147.91 97.75) (width 0.15) (layer F.Cu) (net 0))
 (segment (start 145.57 100.09) (end 145.57 101.91) (width 0.15) (layer F.Cu) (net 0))
 (segment (start 145.57 101.91) (end 145.57 101.98) (width 0.15) (layer F.Cu) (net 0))
 (segment (start 147.91 97.75) (end 145.57 100.09) (width 0.15) (layer F.Cu) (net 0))
 (segment (start 148.55 98.25) (end 147.91 98.25) (width 0.15) (layer F.Cu) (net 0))
 (segment (start 145.92 100.24) (end 145.92 101.99) (width 0.15) (layer F.Cu) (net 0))
 (segment (start 145.92 101.99) (end 145.92 102.02) (width 0.15) (layer F.Cu) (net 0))
 (segment (start 147.91 98.25) (end 145.92 100.24) (width 0.15) (layer F.Cu) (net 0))
 (segment (start 148.55 98.75) (end 147.91 98.75) (width 0.15) (layer F.Cu) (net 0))
 (segment (start 146.27 100.39) (end 146.27 101.95) (width 0.15) (layer F.Cu) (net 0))
 (segment (start 146.27 101.95) (end 146.27 101.98) (width 0.15) (layer F.Cu) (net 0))
 (segment (start 147.91 98.75) (end 146.27 100.39) (width 0.15) (layer F.Cu) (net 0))
 (segment (start 148.55 99.25) (end 147.91 99.25) (width 0.15) (layer F.Cu) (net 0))
 (segment (start 146.62 100.54) (end 146.62 101.85) (width 0.15) (layer F.Cu) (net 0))
 (segment (start 146.62 101.85) (end 146.62 101.92) (width 0.15) (layer F.Cu) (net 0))
 (segment (start 147.91 99.25) (end 146.62 100.54) (width 0.15) (layer F.Cu) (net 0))
 (segment (start 148.55 99.75) (end 147.91 99.75) (width 0.15) (layer F.Cu) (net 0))
 (segment (start 146.97 100.69) (end 146.97 101.78) (width 0.15) (layer F.Cu) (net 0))
 (segment (start 146.97 101.78) (end 146.97 101.87) (width 0.15) (layer F.Cu) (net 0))
 (segment (start 147.91 99.75) (end 146.97 100.69) (width 0.15) (layer F.Cu) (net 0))
 (segment (start 148.55 100.75) (end 147.91 100.75) (width 0.15) (layer F.Cu) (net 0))
 (segment (start 147.67 100.99) (end 147.67 101.9) (width 0.15) (layer F.Cu) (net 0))
 (segment (start 147.67 101.9) (end 147.67 101.93) (width 0.15) (layer F.Cu) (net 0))
 (segment (start 147.91 100.75) (end 147.67 100.99) (width 0.15) (layer F.Cu) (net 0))
 (segment (start 150.05 102.75) (end 150.05 127.71) (width 0.15) (layer F.Cu) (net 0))
 (segment (start 150.27 127.71) (end 162.38 127.71) (width 0.15) (layer F.Cu) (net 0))
 (segment (start 150.05 127.71) (end 150.27 127.71) (width 0.15) (layer F.Cu) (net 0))
 (segment (start 150.55 102.75) (end 150.55 125.17) (width 0.15) (layer F.Cu) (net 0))
 (segment (start 150.87 125.17) (end 162.38 125.17) (width 0.15) (layer F.Cu) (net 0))
 (segment (start 150.55 125.17) (end 150.87 125.17) (width 0.15) (layer F.Cu) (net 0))
 (segment (start 151.05 102.75) (end 151.05 122.63) (width 0.15) (layer F.Cu) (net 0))
 (segment (start 151.33 122.63) (end 162.38 122.63) (width 0.15) (layer F.Cu) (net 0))
 (segment (start 151.05 122.63) (end 151.33 122.63) (width 0.15) (layer F.Cu) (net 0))
 (segment (start 151.55 102.75) (end 151.55 120.09) (width 0.15) (layer F.Cu) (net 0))
 (segment (start 151.65 120.09) (end 162.38 120.09) (width 0.15) (layer F.Cu) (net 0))
 (segment (start 151.55 120.09) (end 151.65 120.09) (width 0.15) (layer F.Cu) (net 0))
 (segment (start 152.05 102.75) (end 152.05 117.55) (width 0.15) (layer F.Cu) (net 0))
 (segment (start 152.32 117.55) (end 162.38 117.55) (width 0.15) (layer F.Cu) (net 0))
 (segment (start 152.05 117.55) (end 152.32 117.55) (width 0.15) (layer F.Cu) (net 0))
 (segment (start 152.55 102.75) (end 152.55 115.01) (width 0.15) (layer F.Cu) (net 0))
 (segment (start 152.85 115.01) (end 162.38 115.01) (width 0.15) (layer F.Cu) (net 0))
 (segment (start 152.55 115.01) (end 152.85 115.01) (width 0.15) (layer F.Cu) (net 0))
 (segment (start 153.05 102.75) (end 153.05 112.47) (width 0.15) (layer F.Cu) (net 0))
 (segment (start 153.39 112.47) (end 162.38 112.47) (width 0.15) (layer F.Cu) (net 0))
 (segment (start 153.05 112.47) (end 153.39 112.47) (width 0.15) (layer F.Cu) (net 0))
 (segment (start 153.55 102.75) (end 153.55 109.93) (width 0.15) (layer F.Cu) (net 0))
 (segment (start 153.82 109.93) (end 162.38 109.93) (width 0.15) (layer F.Cu) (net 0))
 (segment (start 153.55 109.93) (end 153.82 109.93) (width 0.15) (layer F.Cu) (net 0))
 (segment (start 154.05 102.75) (end 154.05 107.39) (width 0.15) (layer F.Cu) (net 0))
 (segment (start 154.3 107.39) (end 162.38 107.39) (width 0.15) (layer F.Cu) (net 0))
 (segment (start 154.05 107.39) (end 154.3 107.39) (width 0.15) (layer F.Cu) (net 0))
 (segment (start 154.55 102.75) (end 154.55 104.85) (width 0.15) (layer F.Cu) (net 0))
 (segment (start 154.86 104.85) (end 162.38 104.85) (width 0.15) (layer F.Cu) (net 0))
 (segment (start 154.55 104.85) (end 154.86 104.85) (width 0.15) (layer F.Cu) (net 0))
 (segment (start 155.05 102.75) (end 155.05 103.39) (width 0.15) (layer F.Cu) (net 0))
 (segment (start 161.06 103.63) (end 162.38 102.31) (width 0.15) (layer F.Cu) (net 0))
 (segment (start 155.29 103.63) (end 161.06 103.63) (width 0.15) (layer F.Cu) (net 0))
 (segment (start 155.05 103.39) (end 155.29 103.63) (width 0.15) (layer F.Cu) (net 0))
 (segment (start 155.55 102.75) (end 159.4 102.75) (width 0.15) (layer F.Cu) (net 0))
 (segment (start 159.4 102.75) (end 162.38 99.77) (width 0.15) (layer F.Cu) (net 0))
 (segment (start 157.05 95.75) (end 157.05 74.62) (width 0.15) (layer F.Cu) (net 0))
 (segment (start 157.05 74.62) (end 162.38 69.29) (width 0.15) (layer F.Cu) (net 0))
 (segment (start 157.93 95.08) (end 157.93 76.28) (width 0.15) (layer F.Cu) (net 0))
 (segment (start 157.93 76.28) (end 162.38 71.83) (width 0.15) (layer F.Cu) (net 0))
 (segment (start 158.28 95.65) (end 158.28 78.47) (width 0.15) (layer F.Cu) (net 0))
 (segment (start 158.28 96.16) (end 158.28 95.65) (width 0.15) (layer F.Cu) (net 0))
 (segment (start 157.69 96.75) (end 158.28 96.16) (width 0.15) (layer F.Cu) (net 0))
 (segment (start 157.05 96.75) (end 157.69 96.75) (width 0.15) (layer F.Cu) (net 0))
 (segment (start 158.28 78.47) (end 162.38 74.37) (width 0.15) (layer F.Cu) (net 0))
 (segment (start 158.63 95.72) (end 158.63 80.66) (width 0.15) (layer F.Cu) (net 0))
 (segment (start 158.63 96.31) (end 158.63 95.72) (width 0.15) (layer F.Cu) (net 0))
 (segment (start 157.69 97.25) (end 158.63 96.31) (width 0.15) (layer F.Cu) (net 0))
 (segment (start 157.05 97.25) (end 157.69 97.25) (width 0.15) (layer F.Cu) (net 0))
 (segment (start 158.63 80.66) (end 162.38 76.91) (width 0.15) (layer F.Cu) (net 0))
 (segment (start 158.98 95.67) (end 158.98 82.85) (width 0.15) (layer F.Cu) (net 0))
 (segment (start 158.98 96.46) (end 158.98 95.67) (width 0.15) (layer F.Cu) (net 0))
 (segment (start 157.69 97.75) (end 158.98 96.46) (width 0.15) (layer F.Cu) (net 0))
 (segment (start 157.05 97.75) (end 157.69 97.75) (width 0.15) (layer F.Cu) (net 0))
 (segment (start 158.98 82.85) (end 162.38 79.45) (width 0.15) (layer F.Cu) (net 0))
 (segment (start 159.33 95.62) (end 159.33 85.04) (width 0.15) (layer F.Cu) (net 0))
 (segment (start 159.33 96.61) (end 159.33 95.62) (width 0.15) (layer F.Cu) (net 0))
 (segment (start 157.69 98.25) (end 159.33 96.61) (width 0.15) (layer F.Cu) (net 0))
 (segment (start 157.05 98.25) (end 157.69 98.25) (width 0.15) (layer F.Cu) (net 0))
 (segment (start 159.33 85.04) (end 162.38 81.99) (width 0.15) (layer F.Cu) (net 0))
 (segment (start 159.68 94.97) (end 159.68 87.23) (width 0.15) (layer F.Cu) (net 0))
 (segment (start 157.05 98.75) (end 157.69 98.75) (width 0.15) (layer F.Cu) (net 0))
 (segment (start 157.69 98.75) (end 159.68 96.76) (width 0.15) (layer F.Cu) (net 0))
 (segment (start 159.68 96.76) (end 159.68 94.97) (width 0.15) (layer F.Cu) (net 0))
 (segment (start 159.68 87.23) (end 162.38 84.53) (width 0.15) (layer F.Cu) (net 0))
 (segment (start 160.03 95.22) (end 160.03 89.42) (width 0.15) (layer F.Cu) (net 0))
 (segment (start 157.05 99.25) (end 157.69 99.25) (width 0.15) (layer F.Cu) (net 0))
 (segment (start 157.69 99.25) (end 160.03 96.91) (width 0.15) (layer F.Cu) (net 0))
 (segment (start 160.03 96.91) (end 160.03 95.22) (width 0.15) (layer F.Cu) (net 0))
 (segment (start 160.03 89.42) (end 162.38 87.07) (width 0.15) (layer F.Cu) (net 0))
 (segment (start 160.38 95.9) (end 160.38 91.61) (width 0.15) (layer F.Cu) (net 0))
 (segment (start 160.38 91.61) (end 162.38 89.61) (width 0.15) (layer F.Cu) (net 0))
 (segment (start 157.05 99.75) (end 157.69 99.75) (width 0.15) (layer F.Cu) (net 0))
 (segment (start 157.69 99.75) (end 160.38 97.06) (width 0.15) (layer F.Cu) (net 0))
 (segment (start 160.38 97.06) (end 160.38 95.9) (width 0.15) (layer F.Cu) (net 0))
 (segment (start 160.38 95.9) (end 160.38 95.85) (width 0.15) (layer F.Cu) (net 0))
 (segment (start 160.73 95.99) (end 160.73 93.8) (width 0.15) (layer F.Cu) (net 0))
 (segment (start 157.05 100.25) (end 157.69 100.25) (width 0.15) (layer F.Cu) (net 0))
 (segment (start 157.69 100.25) (end 160.73 97.21) (width 0.15) (layer F.Cu) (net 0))
 (segment (start 160.73 97.21) (end 160.73 95.99) (width 0.15) (layer F.Cu) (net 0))
 (segment (start 160.73 93.8) (end 162.38 92.15) (width 0.15) (layer F.Cu) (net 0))
 (segment (start 161.08 96.38) (end 161.08 95.99) (width 0.15) (layer F.Cu) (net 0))
 (segment (start 157.05 100.75) (end 157.69 100.75) (width 0.15) (layer F.Cu) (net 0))
 (segment (start 157.69 100.75) (end 161.08 97.36) (width 0.15) (layer F.Cu) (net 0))
 (segment (start 161.08 97.36) (end 161.08 96.38) (width 0.15) (layer F.Cu) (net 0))
 (segment (start 161.08 95.99) (end 162.38 94.69) (width 0.15) (layer F.Cu) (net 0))
 (segment (start 157.05 101.25) (end 157.69 101.25) (width 0.15) (layer F.Cu) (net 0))
 (segment (start 157.69 101.25) (end 161.71 97.23) (width 0.15) (layer F.Cu) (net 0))
 (segment (start 161.71 97.23) (end 162.38 97.23) (width 0.15) (layer F.Cu) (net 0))
 (segment (start 157.05 96.25) (end 157.69 96.25) (width 0.15) (layer F.Cu) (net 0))
 (segment (start 157.69 96.25) (end 157.93 96.01) (width 0.15) (layer F.Cu) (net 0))
 (segment (start 157.93 96.01) (end 157.93 95.08) (width 0.15) (layer F.Cu) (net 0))
 (segment (start 157.93 95.08) (end 157.93 95.06) (width 0.15) (layer F.Cu) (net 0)))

